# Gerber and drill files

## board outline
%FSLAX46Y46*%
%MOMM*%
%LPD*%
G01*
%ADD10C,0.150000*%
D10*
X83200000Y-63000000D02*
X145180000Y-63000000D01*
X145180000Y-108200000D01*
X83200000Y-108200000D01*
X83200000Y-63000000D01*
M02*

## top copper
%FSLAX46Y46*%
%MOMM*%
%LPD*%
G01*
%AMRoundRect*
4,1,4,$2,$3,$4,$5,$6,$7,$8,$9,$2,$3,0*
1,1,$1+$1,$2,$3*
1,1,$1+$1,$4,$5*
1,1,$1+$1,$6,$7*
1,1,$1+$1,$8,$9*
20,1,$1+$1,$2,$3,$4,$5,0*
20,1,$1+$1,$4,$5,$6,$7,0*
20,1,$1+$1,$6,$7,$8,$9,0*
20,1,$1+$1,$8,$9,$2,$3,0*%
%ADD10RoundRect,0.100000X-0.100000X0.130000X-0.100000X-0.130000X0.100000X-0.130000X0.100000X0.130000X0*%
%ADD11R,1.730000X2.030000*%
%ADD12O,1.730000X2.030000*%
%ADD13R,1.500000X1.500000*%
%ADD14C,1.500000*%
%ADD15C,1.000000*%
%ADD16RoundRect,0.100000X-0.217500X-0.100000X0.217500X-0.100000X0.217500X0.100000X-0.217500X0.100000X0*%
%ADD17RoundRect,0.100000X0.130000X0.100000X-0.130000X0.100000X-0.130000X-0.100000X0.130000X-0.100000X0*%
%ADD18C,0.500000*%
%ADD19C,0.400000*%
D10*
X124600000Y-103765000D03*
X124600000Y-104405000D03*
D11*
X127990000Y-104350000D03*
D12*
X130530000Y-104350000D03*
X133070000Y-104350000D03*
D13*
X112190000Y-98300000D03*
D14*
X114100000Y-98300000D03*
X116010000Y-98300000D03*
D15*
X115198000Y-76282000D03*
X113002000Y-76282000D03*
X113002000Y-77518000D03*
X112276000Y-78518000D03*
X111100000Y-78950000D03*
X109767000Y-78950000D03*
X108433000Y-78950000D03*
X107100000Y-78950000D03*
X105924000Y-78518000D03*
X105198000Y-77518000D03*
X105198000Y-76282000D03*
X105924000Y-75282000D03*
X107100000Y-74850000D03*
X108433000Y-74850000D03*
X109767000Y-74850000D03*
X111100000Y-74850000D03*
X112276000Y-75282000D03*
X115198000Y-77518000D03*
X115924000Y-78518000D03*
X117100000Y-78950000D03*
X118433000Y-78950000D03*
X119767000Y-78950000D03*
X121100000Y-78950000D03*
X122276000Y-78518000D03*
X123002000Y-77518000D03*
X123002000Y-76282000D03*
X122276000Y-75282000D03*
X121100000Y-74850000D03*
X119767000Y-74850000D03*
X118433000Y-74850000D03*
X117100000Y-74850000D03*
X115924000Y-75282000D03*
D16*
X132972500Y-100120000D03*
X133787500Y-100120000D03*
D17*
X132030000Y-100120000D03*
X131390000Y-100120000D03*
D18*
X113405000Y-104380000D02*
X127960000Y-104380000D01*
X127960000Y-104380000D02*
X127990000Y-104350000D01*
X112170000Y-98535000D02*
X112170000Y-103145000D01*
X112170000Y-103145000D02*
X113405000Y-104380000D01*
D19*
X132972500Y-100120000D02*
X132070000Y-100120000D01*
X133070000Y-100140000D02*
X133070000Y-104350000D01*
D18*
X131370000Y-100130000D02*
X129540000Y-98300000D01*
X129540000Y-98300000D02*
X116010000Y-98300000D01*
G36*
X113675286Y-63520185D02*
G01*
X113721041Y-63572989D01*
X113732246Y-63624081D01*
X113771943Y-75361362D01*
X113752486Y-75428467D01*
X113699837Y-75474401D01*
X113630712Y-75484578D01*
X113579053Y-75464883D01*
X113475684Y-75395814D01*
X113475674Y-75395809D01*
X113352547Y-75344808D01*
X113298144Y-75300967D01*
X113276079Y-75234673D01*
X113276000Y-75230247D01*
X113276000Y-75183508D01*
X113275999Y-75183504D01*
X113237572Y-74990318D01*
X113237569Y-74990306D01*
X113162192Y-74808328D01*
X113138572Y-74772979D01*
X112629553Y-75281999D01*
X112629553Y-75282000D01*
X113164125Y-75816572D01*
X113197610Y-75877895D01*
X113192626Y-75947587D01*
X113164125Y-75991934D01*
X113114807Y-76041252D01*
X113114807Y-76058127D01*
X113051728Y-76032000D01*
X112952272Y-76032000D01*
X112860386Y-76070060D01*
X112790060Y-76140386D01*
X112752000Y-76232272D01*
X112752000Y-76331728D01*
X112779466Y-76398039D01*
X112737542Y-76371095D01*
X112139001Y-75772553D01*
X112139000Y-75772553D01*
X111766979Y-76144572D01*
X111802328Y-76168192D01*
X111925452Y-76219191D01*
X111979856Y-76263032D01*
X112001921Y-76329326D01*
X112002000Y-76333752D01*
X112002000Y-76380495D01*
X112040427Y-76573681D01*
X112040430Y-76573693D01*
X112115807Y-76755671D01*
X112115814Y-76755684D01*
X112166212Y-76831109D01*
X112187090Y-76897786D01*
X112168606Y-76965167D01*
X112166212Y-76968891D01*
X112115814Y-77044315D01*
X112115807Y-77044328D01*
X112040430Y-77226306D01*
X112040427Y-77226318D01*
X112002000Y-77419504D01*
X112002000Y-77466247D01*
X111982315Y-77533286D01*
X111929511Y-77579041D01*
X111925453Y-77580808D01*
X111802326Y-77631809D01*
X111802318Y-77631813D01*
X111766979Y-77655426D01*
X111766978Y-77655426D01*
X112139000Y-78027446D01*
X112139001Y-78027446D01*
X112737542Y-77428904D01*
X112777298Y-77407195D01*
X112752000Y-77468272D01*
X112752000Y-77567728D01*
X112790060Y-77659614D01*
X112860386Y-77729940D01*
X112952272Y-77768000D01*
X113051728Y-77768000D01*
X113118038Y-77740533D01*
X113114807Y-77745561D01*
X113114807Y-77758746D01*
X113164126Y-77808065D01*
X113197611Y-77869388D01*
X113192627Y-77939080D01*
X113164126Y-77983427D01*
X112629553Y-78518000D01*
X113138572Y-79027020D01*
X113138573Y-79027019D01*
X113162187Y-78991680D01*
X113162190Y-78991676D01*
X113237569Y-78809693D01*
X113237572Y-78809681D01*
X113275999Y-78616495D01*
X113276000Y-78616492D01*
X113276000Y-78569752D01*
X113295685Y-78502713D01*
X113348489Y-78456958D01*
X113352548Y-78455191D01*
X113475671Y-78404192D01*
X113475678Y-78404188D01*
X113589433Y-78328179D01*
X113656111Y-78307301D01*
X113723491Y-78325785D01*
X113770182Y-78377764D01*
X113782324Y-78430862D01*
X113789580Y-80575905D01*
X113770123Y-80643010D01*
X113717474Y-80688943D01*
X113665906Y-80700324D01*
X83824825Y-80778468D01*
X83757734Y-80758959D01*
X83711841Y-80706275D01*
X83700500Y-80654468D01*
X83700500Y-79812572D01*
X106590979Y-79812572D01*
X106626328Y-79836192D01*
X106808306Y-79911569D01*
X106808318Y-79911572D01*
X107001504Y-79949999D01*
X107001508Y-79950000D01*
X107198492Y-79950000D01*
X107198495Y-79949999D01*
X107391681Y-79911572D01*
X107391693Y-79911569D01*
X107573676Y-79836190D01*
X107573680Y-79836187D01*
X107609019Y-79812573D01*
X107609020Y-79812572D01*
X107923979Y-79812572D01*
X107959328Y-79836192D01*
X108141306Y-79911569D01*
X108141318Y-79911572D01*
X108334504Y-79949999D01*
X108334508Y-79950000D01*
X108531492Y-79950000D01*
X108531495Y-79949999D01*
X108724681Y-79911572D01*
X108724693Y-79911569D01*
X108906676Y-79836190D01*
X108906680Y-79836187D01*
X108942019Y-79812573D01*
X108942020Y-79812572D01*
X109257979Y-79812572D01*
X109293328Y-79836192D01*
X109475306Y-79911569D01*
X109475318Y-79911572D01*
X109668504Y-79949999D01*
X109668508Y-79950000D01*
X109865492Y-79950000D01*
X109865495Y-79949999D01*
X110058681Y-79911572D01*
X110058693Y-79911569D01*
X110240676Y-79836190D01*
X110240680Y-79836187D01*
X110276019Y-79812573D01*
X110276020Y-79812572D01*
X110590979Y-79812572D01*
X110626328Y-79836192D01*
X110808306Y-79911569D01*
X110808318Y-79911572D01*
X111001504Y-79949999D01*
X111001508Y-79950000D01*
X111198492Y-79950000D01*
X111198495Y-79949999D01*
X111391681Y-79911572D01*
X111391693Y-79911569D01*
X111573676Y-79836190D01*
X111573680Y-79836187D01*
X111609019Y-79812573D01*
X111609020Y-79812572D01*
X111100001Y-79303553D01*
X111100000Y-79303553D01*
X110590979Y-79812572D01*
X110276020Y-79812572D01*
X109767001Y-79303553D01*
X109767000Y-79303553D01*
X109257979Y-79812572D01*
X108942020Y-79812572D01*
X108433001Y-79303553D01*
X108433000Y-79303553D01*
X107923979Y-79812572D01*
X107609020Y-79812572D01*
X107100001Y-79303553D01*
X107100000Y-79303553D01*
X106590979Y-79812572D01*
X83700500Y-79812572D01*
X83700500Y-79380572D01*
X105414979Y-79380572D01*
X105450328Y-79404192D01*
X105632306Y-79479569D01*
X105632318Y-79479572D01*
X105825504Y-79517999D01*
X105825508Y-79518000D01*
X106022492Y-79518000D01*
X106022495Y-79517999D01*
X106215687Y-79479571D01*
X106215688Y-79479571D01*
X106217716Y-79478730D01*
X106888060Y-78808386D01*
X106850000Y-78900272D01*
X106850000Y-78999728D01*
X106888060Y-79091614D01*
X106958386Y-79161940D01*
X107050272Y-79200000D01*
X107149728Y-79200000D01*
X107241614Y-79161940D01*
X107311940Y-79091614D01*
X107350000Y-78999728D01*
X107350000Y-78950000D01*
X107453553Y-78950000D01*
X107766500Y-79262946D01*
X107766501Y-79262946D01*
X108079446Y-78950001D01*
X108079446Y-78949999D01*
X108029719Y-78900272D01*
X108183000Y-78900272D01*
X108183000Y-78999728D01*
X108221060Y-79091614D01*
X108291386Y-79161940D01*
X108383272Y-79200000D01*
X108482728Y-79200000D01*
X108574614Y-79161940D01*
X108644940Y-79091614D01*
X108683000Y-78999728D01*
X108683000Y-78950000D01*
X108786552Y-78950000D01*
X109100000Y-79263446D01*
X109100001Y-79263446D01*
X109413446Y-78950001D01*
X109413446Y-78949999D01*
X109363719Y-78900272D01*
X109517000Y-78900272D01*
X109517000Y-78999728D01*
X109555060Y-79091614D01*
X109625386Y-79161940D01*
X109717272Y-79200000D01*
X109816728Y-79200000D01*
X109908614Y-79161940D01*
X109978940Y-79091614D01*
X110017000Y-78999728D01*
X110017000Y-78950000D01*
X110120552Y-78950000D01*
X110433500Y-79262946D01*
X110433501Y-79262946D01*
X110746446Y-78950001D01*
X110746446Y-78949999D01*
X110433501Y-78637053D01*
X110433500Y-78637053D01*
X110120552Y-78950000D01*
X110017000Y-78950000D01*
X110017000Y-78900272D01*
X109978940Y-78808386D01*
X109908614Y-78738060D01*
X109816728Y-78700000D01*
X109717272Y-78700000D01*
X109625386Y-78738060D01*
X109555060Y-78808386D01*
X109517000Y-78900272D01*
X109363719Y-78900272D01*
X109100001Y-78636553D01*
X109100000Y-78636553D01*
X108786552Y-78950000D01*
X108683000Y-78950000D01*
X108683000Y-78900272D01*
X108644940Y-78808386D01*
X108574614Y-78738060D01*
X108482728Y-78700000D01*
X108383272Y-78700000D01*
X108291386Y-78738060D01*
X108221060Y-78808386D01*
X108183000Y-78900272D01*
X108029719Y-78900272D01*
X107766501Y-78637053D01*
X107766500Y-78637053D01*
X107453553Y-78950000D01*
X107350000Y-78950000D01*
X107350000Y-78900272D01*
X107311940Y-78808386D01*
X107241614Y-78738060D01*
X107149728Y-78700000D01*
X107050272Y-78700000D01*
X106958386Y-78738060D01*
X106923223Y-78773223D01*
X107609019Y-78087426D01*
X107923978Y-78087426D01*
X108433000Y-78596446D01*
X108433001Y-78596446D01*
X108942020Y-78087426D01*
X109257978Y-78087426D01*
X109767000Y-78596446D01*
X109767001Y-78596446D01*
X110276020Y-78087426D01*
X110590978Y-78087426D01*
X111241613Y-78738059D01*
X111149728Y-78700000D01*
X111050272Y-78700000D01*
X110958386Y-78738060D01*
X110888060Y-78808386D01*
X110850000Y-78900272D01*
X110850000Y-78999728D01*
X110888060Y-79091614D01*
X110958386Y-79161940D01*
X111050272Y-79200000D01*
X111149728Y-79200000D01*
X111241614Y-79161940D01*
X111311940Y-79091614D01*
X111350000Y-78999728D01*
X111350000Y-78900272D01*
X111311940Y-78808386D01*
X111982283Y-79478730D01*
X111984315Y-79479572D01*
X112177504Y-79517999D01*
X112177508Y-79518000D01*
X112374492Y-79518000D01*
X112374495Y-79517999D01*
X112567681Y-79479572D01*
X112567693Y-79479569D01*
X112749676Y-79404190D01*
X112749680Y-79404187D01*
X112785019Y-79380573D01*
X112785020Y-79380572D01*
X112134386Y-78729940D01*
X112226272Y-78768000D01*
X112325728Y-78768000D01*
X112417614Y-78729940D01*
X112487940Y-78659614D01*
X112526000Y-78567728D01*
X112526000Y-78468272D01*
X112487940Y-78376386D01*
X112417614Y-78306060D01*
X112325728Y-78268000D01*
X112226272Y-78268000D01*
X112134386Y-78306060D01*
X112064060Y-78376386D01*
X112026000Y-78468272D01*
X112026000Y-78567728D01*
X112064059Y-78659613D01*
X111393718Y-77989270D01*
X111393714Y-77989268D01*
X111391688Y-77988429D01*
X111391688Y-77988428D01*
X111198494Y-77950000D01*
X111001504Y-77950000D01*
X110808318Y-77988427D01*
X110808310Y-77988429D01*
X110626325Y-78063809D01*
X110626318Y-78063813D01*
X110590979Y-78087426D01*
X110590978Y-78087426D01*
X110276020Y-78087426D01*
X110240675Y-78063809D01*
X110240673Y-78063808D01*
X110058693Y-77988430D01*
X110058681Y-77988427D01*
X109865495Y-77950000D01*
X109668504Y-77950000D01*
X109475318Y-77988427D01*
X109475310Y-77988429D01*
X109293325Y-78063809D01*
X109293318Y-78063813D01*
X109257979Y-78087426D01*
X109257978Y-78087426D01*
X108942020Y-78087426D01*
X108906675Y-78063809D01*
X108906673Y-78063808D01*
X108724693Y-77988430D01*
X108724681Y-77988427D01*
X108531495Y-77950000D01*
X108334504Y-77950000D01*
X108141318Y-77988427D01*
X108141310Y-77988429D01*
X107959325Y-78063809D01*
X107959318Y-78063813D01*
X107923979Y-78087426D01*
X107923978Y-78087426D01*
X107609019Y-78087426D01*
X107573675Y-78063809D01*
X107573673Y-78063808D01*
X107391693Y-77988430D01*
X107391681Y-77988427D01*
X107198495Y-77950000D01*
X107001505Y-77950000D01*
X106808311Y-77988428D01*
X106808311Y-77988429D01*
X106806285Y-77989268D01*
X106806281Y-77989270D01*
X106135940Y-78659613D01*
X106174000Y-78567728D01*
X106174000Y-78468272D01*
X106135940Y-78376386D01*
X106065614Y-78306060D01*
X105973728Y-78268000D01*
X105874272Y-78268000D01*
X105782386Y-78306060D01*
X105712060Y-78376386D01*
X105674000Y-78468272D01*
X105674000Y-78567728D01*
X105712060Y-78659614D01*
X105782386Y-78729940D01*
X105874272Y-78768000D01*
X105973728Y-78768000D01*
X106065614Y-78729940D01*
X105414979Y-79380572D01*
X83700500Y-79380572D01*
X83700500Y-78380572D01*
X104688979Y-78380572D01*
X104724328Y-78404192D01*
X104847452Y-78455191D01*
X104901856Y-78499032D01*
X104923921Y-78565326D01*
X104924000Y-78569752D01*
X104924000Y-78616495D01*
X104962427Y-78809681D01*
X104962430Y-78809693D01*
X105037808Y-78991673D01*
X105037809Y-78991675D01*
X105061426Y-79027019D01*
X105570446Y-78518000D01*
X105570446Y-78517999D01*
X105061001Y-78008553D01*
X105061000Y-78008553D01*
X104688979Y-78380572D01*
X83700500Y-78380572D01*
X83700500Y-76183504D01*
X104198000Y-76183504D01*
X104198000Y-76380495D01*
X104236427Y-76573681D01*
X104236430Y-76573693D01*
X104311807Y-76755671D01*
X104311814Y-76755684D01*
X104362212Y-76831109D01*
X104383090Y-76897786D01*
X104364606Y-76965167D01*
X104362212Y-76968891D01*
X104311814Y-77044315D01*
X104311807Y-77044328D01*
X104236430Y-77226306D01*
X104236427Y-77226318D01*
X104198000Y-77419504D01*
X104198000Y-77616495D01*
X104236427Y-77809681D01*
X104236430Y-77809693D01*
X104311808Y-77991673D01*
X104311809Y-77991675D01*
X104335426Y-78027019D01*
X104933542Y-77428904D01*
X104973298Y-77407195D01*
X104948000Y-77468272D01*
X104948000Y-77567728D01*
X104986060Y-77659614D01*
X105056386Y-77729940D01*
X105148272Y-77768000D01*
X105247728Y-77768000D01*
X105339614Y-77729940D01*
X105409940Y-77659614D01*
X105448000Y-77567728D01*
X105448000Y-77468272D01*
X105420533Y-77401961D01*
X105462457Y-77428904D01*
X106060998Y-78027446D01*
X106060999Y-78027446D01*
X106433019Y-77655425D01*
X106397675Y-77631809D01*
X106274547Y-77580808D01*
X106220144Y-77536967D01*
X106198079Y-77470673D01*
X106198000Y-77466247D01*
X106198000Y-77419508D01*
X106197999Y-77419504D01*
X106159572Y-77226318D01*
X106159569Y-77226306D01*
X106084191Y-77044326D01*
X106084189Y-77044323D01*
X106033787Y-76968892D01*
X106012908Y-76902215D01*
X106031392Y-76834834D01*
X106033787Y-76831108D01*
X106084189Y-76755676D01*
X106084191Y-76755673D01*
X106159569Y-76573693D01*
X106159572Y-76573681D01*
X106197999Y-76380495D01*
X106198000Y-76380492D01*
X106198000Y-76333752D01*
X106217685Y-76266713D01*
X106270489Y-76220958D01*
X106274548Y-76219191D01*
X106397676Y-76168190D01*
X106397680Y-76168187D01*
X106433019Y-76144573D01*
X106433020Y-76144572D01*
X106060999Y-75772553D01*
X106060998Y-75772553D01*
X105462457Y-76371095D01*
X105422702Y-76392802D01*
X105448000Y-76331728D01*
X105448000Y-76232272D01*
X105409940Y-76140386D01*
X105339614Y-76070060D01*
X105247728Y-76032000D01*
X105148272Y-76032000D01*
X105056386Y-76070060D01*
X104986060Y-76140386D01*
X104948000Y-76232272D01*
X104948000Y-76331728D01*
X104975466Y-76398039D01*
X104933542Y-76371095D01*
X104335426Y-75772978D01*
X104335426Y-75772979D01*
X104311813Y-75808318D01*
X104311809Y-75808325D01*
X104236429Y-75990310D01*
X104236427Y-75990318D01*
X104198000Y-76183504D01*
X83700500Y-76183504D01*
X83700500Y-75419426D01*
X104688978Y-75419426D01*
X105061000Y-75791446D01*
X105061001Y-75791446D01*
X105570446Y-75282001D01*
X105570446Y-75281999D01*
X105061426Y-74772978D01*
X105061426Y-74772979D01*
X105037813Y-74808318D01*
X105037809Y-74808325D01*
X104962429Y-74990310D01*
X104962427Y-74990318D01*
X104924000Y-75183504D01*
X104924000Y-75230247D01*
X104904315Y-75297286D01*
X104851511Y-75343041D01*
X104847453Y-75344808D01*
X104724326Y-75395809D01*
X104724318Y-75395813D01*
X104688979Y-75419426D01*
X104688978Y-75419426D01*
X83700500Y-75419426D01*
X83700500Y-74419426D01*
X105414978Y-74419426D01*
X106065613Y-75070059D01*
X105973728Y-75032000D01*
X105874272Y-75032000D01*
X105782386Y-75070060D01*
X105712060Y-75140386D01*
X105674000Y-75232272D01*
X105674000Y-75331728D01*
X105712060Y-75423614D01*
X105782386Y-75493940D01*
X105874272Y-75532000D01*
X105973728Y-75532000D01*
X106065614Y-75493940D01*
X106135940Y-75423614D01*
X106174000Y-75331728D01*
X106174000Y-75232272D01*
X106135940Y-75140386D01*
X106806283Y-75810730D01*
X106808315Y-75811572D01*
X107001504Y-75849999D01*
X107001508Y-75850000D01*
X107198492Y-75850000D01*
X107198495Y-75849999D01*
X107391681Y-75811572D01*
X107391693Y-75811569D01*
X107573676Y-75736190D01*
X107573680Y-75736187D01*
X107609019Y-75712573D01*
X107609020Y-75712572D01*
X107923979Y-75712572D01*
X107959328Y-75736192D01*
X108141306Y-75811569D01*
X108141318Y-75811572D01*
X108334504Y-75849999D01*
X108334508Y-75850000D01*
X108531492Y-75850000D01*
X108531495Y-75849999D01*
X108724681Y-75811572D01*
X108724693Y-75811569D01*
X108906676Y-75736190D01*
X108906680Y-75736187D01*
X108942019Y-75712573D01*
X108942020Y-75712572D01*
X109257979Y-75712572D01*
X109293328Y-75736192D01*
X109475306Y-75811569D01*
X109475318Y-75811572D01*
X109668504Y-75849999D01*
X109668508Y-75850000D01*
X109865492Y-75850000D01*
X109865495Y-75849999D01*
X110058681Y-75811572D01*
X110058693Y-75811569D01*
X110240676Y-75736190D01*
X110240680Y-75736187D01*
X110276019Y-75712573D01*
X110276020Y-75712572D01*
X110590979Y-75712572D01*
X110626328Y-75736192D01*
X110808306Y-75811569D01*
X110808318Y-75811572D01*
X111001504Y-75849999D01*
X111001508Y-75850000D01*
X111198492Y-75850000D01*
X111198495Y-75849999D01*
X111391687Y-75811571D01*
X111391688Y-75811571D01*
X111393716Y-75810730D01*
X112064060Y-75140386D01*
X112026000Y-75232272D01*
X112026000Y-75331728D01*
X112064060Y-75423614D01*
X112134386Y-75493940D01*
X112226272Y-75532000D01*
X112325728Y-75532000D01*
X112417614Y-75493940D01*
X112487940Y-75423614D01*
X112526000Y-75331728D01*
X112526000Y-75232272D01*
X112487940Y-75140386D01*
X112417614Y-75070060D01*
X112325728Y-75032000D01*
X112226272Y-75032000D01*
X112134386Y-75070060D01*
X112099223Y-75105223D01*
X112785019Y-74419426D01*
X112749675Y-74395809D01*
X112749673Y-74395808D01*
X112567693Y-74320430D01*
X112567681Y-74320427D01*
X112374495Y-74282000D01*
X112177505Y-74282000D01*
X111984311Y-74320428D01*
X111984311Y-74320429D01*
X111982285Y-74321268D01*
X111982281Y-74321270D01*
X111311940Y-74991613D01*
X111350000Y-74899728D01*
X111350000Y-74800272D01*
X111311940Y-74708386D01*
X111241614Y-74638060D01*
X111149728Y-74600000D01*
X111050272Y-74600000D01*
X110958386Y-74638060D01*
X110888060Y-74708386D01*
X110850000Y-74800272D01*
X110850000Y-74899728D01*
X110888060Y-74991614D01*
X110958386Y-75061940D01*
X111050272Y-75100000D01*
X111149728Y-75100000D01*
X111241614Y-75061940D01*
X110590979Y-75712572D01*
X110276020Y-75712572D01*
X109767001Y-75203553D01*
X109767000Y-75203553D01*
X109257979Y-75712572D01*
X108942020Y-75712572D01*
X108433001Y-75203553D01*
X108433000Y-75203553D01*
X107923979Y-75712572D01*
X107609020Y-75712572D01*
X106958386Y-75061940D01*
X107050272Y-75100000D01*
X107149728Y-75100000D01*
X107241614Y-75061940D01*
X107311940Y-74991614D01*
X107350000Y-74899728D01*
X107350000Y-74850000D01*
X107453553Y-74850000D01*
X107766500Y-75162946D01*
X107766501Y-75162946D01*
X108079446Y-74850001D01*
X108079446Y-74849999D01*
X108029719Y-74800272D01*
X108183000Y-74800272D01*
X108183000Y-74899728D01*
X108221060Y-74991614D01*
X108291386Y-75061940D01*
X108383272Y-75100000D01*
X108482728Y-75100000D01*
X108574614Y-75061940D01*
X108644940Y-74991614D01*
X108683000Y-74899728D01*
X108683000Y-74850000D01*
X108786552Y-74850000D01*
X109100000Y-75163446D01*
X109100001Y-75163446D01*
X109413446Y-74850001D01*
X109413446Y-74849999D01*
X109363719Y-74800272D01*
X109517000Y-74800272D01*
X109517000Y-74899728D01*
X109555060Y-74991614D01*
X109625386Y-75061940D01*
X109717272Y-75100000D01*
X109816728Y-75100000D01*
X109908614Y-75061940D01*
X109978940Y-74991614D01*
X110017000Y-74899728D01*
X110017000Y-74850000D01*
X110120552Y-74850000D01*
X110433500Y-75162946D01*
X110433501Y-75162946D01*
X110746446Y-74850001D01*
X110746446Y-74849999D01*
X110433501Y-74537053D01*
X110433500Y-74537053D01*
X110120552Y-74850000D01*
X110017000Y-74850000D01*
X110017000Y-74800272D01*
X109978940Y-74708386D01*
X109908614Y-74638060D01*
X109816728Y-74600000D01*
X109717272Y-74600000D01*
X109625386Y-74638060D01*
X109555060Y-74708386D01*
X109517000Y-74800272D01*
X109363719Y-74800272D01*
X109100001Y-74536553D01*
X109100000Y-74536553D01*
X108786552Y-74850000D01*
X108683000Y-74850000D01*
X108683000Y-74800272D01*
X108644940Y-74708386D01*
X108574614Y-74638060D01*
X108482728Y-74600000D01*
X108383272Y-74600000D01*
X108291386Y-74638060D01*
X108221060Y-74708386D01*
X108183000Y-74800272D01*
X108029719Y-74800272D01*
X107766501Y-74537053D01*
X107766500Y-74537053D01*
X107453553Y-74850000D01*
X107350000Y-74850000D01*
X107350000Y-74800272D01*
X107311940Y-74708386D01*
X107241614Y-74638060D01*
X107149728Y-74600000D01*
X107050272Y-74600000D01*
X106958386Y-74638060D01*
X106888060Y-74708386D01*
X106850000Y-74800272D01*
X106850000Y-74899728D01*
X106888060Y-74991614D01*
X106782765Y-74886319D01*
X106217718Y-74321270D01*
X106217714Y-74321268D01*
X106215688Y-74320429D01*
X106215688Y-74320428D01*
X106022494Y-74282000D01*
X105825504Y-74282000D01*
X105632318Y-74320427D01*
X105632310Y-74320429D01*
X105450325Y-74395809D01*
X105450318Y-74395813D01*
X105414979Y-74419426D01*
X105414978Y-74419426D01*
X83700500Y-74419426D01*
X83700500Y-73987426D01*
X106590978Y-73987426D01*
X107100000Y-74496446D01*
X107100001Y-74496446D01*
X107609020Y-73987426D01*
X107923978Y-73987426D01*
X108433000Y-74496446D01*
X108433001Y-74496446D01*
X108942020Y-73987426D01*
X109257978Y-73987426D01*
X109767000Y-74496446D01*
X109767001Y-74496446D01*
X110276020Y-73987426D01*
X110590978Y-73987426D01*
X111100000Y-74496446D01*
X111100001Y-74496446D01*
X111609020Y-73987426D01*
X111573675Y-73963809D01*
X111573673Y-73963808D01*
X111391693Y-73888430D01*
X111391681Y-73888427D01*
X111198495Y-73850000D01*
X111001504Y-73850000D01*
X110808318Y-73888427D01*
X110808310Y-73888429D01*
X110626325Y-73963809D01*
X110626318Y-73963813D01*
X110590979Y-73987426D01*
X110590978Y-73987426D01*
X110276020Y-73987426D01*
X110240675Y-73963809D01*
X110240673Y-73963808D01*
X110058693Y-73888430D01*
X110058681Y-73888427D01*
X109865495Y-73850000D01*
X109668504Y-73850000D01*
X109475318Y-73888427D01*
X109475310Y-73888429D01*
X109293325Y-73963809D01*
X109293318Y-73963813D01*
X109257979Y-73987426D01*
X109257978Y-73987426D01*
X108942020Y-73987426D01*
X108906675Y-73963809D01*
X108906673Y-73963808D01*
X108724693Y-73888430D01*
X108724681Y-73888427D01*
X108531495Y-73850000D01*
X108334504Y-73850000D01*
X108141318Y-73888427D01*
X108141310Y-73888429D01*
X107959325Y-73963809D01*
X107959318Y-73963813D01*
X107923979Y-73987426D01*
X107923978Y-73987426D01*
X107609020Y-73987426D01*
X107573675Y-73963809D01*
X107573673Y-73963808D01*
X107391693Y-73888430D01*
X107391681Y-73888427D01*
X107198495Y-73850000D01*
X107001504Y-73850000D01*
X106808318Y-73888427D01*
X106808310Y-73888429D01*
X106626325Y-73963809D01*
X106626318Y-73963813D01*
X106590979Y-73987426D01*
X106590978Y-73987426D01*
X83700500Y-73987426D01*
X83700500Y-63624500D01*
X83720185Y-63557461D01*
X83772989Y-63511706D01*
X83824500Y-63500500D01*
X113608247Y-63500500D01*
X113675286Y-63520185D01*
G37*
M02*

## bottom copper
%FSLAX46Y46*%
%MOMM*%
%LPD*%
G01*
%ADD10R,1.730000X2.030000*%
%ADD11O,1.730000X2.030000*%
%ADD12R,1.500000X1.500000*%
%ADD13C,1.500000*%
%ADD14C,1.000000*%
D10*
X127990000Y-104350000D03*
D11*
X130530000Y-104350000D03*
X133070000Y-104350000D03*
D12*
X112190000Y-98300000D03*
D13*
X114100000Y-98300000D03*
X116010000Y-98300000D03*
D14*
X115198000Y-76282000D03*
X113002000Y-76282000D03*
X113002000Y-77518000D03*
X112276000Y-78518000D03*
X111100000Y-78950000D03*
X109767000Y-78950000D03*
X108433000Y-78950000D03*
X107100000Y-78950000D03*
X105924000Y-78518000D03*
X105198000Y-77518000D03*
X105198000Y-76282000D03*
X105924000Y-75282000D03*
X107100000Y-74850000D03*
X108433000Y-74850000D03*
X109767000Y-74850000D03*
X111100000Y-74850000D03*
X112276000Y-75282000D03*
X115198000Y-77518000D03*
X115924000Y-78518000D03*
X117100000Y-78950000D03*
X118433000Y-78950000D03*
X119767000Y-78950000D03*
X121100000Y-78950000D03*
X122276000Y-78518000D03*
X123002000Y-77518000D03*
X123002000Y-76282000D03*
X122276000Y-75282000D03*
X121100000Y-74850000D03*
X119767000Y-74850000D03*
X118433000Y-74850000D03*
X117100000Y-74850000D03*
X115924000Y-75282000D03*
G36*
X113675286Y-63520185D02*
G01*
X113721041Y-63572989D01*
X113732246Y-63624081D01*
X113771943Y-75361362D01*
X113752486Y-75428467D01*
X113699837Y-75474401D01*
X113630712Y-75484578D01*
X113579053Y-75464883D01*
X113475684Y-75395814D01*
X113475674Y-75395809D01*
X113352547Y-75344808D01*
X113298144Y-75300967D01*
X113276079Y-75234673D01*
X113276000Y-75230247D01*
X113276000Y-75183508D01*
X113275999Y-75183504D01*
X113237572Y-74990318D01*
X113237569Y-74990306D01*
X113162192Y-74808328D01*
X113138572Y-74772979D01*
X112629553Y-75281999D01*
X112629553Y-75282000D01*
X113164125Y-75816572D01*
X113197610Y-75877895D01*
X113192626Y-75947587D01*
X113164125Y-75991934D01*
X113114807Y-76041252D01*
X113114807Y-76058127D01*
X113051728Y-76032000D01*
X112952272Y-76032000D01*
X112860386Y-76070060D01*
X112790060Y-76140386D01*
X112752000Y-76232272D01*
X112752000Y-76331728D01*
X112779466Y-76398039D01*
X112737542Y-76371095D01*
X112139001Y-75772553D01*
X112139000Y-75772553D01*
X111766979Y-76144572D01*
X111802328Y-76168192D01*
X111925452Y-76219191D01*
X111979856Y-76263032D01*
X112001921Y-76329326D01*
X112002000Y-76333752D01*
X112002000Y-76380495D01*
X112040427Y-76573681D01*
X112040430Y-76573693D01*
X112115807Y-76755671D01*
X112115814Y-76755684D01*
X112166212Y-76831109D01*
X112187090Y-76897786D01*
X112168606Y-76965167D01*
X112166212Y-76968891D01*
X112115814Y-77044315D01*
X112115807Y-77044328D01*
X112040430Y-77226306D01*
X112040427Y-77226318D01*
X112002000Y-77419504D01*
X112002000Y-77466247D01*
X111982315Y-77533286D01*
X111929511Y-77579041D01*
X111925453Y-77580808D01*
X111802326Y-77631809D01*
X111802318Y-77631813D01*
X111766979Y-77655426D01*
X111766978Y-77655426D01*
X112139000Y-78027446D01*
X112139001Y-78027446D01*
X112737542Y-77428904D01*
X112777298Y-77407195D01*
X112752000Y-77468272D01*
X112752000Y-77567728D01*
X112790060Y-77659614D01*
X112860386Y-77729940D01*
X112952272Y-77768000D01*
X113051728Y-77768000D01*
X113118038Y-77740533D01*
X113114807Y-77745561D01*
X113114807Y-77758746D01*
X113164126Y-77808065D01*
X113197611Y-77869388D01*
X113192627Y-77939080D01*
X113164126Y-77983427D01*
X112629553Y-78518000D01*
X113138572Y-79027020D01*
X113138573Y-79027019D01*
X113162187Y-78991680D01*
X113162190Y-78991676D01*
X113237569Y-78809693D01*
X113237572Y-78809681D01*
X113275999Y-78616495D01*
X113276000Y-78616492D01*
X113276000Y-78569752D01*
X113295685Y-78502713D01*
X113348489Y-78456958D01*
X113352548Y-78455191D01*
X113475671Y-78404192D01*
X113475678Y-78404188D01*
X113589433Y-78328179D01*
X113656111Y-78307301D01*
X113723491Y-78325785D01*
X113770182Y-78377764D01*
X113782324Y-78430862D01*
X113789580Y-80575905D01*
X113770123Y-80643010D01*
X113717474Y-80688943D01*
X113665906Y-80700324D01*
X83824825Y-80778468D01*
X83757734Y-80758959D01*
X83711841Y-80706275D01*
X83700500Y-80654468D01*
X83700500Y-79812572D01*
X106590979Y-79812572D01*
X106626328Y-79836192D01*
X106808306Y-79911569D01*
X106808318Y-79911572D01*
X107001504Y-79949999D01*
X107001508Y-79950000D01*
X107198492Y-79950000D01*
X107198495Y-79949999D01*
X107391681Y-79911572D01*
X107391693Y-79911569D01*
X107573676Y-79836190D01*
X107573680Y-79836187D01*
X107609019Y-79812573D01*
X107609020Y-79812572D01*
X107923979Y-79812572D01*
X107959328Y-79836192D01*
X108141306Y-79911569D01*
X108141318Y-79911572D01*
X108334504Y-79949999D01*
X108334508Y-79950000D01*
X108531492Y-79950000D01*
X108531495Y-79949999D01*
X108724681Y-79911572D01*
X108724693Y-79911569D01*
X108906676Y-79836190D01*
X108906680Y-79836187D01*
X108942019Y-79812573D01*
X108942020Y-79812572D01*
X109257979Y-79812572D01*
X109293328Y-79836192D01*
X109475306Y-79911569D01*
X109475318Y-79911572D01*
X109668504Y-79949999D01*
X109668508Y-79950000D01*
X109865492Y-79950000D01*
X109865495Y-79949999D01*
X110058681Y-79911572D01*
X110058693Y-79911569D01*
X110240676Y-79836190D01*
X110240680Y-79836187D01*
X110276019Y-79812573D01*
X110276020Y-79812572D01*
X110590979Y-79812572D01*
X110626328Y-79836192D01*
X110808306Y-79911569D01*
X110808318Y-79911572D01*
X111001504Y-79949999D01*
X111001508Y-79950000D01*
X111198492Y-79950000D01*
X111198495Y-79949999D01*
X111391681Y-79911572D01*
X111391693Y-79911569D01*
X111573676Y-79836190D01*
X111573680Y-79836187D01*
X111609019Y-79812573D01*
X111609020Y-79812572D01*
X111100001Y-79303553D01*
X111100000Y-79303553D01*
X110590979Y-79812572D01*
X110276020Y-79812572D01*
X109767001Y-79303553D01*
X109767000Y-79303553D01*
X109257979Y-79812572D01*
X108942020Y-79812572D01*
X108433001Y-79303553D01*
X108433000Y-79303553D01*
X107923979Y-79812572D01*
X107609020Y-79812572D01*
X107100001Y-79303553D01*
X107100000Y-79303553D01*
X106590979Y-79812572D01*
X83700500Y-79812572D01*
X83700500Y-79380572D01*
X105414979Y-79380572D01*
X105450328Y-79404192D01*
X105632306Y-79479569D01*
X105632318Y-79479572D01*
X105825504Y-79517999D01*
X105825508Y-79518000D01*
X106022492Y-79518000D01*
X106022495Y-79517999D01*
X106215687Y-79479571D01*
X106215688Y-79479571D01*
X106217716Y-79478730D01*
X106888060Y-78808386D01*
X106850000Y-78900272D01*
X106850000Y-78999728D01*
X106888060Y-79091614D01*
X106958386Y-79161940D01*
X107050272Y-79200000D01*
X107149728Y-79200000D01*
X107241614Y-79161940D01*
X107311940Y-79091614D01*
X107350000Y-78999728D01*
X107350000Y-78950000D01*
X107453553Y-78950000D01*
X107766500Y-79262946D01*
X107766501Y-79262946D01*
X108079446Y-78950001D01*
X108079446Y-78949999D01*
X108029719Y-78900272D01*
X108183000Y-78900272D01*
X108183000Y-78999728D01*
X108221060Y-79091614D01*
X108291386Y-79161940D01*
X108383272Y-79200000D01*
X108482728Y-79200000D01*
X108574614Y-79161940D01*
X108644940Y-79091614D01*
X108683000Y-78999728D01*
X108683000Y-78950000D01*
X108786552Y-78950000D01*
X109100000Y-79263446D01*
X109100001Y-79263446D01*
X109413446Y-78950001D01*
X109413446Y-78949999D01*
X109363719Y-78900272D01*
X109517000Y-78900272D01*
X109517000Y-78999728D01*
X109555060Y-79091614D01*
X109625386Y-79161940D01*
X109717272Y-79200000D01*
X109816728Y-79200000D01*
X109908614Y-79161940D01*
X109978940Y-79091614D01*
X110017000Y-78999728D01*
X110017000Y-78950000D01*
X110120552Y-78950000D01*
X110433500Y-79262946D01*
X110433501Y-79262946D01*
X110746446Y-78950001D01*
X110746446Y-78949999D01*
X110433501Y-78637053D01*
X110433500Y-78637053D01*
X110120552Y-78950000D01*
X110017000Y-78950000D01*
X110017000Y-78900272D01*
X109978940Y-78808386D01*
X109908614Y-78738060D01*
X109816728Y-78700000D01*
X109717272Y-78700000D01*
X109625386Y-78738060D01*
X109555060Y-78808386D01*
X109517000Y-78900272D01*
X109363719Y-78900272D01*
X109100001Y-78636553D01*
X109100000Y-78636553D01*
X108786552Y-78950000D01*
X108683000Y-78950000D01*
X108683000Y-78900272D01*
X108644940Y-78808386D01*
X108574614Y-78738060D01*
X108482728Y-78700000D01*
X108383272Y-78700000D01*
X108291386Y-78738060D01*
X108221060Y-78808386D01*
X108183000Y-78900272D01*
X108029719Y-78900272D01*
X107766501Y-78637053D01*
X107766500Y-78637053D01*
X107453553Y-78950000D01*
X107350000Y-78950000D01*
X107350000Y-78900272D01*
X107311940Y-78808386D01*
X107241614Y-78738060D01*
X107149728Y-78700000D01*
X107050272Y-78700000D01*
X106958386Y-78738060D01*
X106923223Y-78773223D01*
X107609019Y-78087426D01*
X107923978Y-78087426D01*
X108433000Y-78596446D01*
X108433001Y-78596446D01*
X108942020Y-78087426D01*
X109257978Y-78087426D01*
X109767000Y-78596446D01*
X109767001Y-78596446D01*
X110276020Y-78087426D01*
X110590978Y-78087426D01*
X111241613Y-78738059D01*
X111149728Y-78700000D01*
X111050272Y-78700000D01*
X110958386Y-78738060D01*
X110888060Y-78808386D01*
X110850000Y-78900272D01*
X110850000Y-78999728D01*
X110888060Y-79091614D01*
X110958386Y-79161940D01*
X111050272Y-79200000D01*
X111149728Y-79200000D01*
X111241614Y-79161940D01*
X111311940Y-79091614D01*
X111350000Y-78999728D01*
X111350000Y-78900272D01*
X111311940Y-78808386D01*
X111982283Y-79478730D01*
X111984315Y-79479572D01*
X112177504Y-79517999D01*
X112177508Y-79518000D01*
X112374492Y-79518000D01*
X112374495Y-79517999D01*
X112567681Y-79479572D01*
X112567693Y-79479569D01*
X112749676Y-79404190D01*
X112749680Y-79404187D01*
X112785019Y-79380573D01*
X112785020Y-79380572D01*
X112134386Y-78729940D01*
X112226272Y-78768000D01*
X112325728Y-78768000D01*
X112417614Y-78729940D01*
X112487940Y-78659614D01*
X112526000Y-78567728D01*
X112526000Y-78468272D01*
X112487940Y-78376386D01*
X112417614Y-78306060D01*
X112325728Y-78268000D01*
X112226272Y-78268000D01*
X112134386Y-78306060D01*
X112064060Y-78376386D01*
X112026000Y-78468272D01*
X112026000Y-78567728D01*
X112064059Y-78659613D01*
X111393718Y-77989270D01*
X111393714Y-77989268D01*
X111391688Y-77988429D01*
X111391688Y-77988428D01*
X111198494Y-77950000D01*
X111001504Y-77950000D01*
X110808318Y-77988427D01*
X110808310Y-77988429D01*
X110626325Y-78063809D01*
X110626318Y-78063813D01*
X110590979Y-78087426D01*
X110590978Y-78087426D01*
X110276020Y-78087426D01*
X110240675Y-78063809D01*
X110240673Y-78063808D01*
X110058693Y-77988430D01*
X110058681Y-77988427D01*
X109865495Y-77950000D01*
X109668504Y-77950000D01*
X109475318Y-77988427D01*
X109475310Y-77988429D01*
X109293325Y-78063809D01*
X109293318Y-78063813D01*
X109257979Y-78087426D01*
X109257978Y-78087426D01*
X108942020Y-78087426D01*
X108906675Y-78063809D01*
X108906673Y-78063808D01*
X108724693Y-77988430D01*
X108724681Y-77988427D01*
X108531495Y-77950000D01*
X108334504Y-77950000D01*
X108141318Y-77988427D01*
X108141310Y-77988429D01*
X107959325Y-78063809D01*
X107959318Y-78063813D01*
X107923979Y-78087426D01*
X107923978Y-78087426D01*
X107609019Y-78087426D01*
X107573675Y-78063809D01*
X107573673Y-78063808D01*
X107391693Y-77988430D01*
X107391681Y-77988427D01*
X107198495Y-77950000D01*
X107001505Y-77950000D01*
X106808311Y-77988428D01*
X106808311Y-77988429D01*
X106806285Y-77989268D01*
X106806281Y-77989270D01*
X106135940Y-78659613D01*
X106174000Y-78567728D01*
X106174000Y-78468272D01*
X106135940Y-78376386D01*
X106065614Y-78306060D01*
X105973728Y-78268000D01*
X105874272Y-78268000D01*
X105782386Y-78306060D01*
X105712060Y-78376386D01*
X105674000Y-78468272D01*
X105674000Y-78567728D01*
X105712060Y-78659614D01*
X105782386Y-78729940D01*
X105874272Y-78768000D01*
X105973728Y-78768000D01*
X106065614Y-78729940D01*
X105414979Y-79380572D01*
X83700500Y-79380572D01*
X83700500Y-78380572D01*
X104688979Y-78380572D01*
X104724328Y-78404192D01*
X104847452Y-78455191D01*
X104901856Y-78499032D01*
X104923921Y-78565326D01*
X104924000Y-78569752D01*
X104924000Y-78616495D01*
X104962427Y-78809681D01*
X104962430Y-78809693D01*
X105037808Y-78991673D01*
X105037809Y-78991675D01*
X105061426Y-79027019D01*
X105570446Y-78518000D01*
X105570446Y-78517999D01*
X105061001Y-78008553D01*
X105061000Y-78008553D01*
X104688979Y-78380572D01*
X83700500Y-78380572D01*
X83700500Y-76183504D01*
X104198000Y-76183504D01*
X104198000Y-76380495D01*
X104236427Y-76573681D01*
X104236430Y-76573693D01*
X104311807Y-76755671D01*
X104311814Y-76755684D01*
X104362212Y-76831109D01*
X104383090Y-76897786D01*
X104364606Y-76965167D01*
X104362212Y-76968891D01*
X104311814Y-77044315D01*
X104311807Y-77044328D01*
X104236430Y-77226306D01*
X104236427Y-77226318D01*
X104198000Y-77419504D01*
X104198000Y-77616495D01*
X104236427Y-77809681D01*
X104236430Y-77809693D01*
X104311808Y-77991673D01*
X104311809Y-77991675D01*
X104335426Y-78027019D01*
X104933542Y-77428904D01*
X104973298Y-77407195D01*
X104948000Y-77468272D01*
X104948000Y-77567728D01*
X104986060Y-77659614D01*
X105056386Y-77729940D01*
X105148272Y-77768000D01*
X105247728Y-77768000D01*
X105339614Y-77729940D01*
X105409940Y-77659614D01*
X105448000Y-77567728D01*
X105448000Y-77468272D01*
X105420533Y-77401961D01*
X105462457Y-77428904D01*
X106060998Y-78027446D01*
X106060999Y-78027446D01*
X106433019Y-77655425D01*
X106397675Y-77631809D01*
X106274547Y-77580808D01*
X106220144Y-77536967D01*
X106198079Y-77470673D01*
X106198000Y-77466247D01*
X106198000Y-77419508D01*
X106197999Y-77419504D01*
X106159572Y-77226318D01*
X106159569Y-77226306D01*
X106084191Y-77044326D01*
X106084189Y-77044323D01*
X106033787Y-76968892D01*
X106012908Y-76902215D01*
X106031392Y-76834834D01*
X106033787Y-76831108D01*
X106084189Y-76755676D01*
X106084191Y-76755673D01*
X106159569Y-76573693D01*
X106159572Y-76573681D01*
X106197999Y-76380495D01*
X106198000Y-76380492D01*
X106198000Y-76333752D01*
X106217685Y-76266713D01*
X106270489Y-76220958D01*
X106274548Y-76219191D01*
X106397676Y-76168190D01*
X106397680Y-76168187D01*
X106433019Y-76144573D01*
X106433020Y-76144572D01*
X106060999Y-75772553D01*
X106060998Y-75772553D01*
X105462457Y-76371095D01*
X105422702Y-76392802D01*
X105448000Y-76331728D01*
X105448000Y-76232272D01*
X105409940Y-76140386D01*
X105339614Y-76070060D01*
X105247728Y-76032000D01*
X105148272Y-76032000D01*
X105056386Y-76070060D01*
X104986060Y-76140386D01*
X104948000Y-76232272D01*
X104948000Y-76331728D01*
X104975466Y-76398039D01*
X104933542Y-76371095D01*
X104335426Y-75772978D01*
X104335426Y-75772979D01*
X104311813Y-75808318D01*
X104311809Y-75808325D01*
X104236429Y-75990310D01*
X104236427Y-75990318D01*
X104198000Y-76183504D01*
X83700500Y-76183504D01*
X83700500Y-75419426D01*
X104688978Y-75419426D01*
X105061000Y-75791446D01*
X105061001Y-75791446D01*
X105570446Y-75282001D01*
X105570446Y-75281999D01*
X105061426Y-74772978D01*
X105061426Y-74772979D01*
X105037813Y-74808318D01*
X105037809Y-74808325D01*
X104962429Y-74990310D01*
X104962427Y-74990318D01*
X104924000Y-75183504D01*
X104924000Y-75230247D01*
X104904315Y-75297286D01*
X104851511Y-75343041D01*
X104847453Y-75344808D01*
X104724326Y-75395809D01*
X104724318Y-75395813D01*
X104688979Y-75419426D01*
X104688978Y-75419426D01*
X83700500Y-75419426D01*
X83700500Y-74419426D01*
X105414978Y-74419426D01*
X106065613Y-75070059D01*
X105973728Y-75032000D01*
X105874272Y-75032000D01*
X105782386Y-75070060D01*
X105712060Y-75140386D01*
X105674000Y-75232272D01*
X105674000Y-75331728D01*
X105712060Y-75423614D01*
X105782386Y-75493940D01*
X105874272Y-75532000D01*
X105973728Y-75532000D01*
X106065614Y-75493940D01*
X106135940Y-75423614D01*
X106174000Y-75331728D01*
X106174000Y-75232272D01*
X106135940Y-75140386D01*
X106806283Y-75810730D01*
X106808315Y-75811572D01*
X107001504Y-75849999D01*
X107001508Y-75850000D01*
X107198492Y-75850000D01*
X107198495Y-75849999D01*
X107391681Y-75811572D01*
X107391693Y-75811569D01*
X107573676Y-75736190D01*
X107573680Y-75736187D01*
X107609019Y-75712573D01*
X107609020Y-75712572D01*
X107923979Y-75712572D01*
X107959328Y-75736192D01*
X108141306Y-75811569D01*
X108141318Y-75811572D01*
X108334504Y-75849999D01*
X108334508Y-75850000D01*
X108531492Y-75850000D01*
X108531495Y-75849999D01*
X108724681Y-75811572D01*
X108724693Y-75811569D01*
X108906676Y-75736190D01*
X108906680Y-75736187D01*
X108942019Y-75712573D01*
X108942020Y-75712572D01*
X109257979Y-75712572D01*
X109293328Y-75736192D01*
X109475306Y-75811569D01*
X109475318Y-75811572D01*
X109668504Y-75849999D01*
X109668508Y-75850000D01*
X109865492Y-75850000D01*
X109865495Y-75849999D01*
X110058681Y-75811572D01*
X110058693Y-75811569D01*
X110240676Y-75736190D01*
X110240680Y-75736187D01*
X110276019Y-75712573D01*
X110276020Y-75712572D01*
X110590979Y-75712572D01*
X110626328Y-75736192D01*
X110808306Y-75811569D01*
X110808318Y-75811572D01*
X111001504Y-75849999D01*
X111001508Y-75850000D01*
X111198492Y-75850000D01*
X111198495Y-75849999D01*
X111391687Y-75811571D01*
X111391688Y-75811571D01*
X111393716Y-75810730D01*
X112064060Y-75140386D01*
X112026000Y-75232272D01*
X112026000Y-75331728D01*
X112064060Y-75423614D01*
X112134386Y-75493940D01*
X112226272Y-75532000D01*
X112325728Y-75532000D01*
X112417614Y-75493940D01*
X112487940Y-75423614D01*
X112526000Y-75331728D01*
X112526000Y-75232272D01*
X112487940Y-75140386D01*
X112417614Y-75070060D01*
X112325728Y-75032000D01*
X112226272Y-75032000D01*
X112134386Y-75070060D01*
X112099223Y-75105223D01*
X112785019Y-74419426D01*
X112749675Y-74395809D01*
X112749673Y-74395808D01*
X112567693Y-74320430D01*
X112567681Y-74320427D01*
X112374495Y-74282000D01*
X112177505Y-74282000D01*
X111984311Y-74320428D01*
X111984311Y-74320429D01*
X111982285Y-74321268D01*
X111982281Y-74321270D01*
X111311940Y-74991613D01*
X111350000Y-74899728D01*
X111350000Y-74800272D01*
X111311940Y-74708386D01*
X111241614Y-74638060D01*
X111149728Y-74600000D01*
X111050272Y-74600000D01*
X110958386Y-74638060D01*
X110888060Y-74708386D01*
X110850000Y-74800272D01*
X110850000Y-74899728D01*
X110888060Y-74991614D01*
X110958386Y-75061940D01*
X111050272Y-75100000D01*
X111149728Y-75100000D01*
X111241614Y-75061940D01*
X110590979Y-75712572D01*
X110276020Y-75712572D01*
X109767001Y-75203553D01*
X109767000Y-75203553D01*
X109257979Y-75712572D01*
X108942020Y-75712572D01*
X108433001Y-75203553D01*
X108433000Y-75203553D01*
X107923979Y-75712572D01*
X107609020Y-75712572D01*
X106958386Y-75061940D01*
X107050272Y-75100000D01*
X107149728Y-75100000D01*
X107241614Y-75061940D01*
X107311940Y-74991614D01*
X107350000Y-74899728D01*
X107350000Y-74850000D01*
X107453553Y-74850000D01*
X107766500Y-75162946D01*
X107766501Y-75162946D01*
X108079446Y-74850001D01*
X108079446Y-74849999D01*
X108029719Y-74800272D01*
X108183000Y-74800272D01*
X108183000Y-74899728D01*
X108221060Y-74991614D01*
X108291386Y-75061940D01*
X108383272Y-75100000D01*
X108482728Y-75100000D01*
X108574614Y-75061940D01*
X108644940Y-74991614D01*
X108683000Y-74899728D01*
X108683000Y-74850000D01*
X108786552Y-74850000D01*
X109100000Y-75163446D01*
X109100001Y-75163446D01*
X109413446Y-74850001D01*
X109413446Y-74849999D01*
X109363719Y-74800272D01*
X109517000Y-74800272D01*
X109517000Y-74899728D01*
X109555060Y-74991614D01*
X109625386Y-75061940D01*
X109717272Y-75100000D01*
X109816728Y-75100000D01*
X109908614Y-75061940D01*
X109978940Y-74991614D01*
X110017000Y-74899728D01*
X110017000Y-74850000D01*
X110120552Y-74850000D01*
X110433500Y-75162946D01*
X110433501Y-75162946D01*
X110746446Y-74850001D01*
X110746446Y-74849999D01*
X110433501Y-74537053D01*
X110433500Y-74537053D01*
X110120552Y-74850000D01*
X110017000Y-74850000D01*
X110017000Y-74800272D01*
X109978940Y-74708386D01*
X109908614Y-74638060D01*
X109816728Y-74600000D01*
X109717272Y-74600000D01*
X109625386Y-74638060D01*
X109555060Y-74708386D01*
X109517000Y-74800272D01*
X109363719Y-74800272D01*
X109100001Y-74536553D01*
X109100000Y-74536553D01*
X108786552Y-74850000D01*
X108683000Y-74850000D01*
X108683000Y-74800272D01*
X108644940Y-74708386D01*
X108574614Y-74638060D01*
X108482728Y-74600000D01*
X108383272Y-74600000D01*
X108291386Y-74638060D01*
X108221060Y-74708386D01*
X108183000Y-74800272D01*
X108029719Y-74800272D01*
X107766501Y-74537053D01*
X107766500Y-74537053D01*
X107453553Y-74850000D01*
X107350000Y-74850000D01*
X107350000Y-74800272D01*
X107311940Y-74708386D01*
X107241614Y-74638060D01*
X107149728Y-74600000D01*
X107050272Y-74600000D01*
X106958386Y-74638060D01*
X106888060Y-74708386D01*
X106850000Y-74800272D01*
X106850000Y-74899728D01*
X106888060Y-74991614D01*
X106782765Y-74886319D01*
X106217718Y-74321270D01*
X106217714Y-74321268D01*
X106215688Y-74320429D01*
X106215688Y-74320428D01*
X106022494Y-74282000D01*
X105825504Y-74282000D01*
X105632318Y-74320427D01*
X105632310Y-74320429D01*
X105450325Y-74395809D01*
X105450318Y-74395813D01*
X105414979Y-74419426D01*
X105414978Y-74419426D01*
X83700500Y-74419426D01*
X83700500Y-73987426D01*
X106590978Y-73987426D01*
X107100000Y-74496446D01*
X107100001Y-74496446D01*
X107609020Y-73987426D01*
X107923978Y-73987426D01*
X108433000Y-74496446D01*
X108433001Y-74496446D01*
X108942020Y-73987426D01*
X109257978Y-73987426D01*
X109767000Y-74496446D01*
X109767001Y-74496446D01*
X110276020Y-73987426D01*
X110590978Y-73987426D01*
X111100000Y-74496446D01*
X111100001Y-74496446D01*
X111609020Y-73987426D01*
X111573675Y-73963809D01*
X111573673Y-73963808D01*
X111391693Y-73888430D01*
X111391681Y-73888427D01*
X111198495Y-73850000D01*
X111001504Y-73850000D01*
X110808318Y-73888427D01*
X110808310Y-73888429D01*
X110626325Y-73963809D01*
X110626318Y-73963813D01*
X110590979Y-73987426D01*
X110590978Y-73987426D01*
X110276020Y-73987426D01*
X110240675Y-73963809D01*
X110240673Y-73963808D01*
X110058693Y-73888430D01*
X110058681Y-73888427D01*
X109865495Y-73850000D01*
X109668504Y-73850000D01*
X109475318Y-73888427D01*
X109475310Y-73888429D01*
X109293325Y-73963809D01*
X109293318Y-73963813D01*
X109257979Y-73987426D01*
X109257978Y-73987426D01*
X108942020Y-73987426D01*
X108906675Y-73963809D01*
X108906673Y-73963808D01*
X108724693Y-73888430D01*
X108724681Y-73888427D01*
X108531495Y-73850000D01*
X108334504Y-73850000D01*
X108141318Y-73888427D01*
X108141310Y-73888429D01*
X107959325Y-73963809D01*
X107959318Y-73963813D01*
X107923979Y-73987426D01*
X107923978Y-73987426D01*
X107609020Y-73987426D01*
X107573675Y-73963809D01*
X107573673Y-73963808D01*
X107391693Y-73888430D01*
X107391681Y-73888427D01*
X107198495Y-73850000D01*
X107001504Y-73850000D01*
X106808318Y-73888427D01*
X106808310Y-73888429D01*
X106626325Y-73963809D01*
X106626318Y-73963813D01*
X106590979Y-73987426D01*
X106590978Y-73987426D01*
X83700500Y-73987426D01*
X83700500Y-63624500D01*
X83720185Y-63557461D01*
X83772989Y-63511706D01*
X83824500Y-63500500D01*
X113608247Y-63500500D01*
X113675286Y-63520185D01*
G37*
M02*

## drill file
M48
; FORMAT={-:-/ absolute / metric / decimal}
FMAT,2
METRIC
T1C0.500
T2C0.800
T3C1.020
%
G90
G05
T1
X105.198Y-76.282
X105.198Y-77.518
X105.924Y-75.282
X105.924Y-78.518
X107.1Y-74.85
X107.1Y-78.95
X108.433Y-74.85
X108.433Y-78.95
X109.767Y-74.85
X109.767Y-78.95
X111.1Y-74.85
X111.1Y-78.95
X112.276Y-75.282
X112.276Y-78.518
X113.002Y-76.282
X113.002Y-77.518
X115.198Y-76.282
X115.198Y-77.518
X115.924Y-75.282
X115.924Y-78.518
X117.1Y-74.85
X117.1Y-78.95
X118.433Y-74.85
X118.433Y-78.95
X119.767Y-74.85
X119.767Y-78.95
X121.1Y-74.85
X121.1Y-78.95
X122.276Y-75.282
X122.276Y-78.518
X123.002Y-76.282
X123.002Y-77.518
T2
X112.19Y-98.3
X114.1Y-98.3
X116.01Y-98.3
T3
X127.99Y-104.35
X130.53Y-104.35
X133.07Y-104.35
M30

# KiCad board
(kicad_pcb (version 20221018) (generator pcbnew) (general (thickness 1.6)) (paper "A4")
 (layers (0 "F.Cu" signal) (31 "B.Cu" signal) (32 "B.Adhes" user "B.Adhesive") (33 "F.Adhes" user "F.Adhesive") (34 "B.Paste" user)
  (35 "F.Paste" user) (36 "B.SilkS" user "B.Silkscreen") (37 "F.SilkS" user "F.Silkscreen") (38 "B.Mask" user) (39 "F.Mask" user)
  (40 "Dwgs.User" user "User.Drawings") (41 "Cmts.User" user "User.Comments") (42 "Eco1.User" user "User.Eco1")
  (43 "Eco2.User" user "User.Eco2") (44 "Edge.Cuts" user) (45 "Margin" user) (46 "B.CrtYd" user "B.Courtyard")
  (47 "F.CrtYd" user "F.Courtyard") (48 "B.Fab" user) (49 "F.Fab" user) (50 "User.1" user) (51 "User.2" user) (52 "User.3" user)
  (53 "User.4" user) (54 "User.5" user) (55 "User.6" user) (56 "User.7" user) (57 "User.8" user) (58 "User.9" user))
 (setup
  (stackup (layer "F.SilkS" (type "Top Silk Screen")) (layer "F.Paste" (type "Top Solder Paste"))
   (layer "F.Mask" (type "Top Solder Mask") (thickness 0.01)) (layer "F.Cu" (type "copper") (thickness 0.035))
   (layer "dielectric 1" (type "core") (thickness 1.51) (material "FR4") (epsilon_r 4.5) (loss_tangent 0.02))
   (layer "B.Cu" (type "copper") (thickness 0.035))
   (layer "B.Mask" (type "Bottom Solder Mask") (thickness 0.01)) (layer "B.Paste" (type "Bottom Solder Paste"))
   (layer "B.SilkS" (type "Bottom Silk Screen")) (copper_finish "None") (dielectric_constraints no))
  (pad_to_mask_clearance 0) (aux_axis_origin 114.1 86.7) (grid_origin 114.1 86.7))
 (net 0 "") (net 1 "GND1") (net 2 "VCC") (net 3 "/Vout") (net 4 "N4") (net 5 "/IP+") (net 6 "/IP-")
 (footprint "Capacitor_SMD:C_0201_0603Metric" (layer "F.Cu") (at 124.6 104.085 -90)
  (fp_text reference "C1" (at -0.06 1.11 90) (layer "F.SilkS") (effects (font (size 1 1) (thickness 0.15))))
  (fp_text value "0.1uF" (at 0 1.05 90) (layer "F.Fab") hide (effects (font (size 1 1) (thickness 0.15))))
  (pad "" smd roundrect (at -0.345 0 270) (size 0.318 0.36) (layers "F.Paste") (roundrect_rratio 0.25))
  (pad "" smd roundrect (at 0.345 0 270) (size 0.318 0.36) (layers "F.Paste") (roundrect_rratio 0.25))
  (pad "1" smd roundrect (at -0.32 0 270) (size 0.46 0.4) (layers "F.Cu" "F.Mask") (roundrect_rratio 0.25) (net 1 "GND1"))
  (pad "2" smd roundrect (at 0.32 0 270) (size 0.46 0.4) (layers "F.Cu" "F.Mask") (roundrect_rratio 0.25) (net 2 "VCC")))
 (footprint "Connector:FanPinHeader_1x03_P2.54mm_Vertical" (layer "F.Cu") (at 127.99 104.35)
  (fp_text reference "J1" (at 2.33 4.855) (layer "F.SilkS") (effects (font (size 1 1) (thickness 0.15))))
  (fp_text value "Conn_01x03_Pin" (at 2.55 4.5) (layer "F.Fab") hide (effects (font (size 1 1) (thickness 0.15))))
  (pad "1" thru_hole rect (at 0 0 90) (size 2.03 1.73) (drill 1.02) (layers "*.Cu" "*.Mask") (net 2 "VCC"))
  (pad "2" thru_hole oval (at 2.54 0 90) (size 2.03 1.73) (drill 1.02) (layers "*.Cu" "*.Mask") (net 1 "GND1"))
  (pad "3" thru_hole oval (at 5.08 0 90) (size 2.03 1.73) (drill 1.02) (layers "*.Cu" "*.Mask") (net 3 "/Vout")))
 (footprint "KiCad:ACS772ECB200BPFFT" (layer "F.Cu") (at 112.19 98.3)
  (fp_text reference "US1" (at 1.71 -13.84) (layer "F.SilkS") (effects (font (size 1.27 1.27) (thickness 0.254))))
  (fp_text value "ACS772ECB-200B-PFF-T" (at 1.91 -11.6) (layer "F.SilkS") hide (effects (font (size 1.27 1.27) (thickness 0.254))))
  (pad "1" thru_hole rect (at 0 0) (size 1.5 1.5) (drill 0.8) (layers "*.Cu" "*.Mask") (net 2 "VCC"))
  (pad "2" thru_hole circle (at 1.91 0) (size 1.5 1.5) (drill 0.8) (layers "*.Cu" "*.Mask") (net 1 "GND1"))
  (pad "3" thru_hole circle (at 3.82 0) (size 1.5 1.5) (drill 0.8) (layers "*.Cu" "*.Mask") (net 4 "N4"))
  (pad "4" thru_hole circle (at 3.008 -22.018) (size 1 1) (drill 0.5) (layers "*.Cu" "*.Mask") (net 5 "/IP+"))
  (pad "5" thru_hole circle (at 0.812 -22.018) (size 1 1) (drill 0.5) (layers "*.Cu" "*.Mask") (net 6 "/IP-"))
  (pad "6" thru_hole circle (at 0.812 -20.782) (size 1 1) (drill 0.5) (layers "*.Cu" "*.Mask") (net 6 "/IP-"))
  (pad "7" thru_hole circle (at 0.086 -19.782) (size 1 1) (drill 0.5) (layers "*.Cu" "*.Mask") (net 6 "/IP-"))
  (pad "8" thru_hole circle (at -1.09 -19.35) (size 1 1) (drill 0.5) (layers "*.Cu" "*.Mask") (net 6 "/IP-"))
  (pad "9" thru_hole circle (at -2.423 -19.35) (size 1 1) (drill 0.5) (layers "*.Cu" "*.Mask") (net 6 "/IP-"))
  (pad "10" thru_hole circle (at -3.757 -19.35) (size 1 1) (drill 0.5) (layers "*.Cu" "*.Mask") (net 6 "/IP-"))
  (pad "11" thru_hole circle (at -5.09 -19.35) (size 1 1) (drill 0.5) (layers "*.Cu" "*.Mask") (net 6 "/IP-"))
  (pad "12" thru_hole circle (at -6.266 -19.782) (size 1 1) (drill 0.5) (layers "*.Cu" "*.Mask") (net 6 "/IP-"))
  (pad "13" thru_hole circle (at -6.992 -20.782) (size 1 1) (drill 0.5) (layers "*.Cu" "*.Mask") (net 6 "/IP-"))
  (pad "14" thru_hole circle (at -6.992 -22.018) (size 1 1) (drill 0.5) (layers "*.Cu" "*.Mask") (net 6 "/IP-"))
  (pad "15" thru_hole circle (at -6.266 -23.018) (size 1 1) (drill 0.5) (layers "*.Cu" "*.Mask") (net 6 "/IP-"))
  (pad "16" thru_hole circle (at -5.09 -23.45) (size 1 1) (drill 0.5) (layers "*.Cu" "*.Mask") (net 6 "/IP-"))
  (pad "17" thru_hole circle (at -3.757 -23.45) (size 1 1) (drill 0.5) (layers "*.Cu" "*.Mask") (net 6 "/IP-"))
  (pad "18" thru_hole circle (at -2.423 -23.45) (size 1 1) (drill 0.5) (layers "*.Cu" "*.Mask") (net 6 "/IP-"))
  (pad "19" thru_hole circle (at -1.09 -23.45) (size 1 1) (drill 0.5) (layers "*.Cu" "*.Mask") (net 6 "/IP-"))
  (pad "20" thru_hole circle (at 0.086 -23.018) (size 1 1) (drill 0.5) (layers "*.Cu" "*.Mask") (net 6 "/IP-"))
  (pad "21" thru_hole circle (at 3.008 -20.782) (size 1 1) (drill 0.5) (layers "*.Cu" "*.Mask") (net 5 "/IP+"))
  (pad "22" thru_hole circle (at 3.734 -19.782) (size 1 1) (drill 0.5) (layers "*.Cu" "*.Mask") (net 5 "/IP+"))
  (pad "23" thru_hole circle (at 4.91 -19.35) (size 1 1) (drill 0.5) (layers "*.Cu" "*.Mask") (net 5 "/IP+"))
  (pad "24" thru_hole circle (at 6.243 -19.35) (size 1 1) (drill 0.5) (layers "*.Cu" "*.Mask") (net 5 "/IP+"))
  (pad "25" thru_hole circle (at 7.577 -19.35) (size 1 1) (drill 0.5) (layers "*.Cu" "*.Mask") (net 5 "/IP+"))
  (pad "26" thru_hole circle (at 8.91 -19.35) (size 1 1) (drill 0.5) (layers "*.Cu" "*.Mask") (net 5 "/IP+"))
  (pad "27" thru_hole circle (at 10.086 -19.782) (size 1 1) (drill 0.5) (layers "*.Cu" "*.Mask") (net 5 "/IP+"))
  (pad "28" thru_hole circle (at 10.812 -20.782) (size 1 1) (drill 0.5) (layers "*.Cu" "*.Mask") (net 5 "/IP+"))
  (pad "29" thru_hole circle (at 10.812 -22.018) (size 1 1) (drill 0.5) (layers "*.Cu" "*.Mask") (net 5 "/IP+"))
  (pad "30" thru_hole circle (at 10.086 -23.018) (size 1 1) (drill 0.5) (layers "*.Cu" "*.Mask") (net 5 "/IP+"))
  (pad "31" thru_hole circle (at 8.91 -23.45) (size 1 1) (drill 0.5) (layers "*.Cu" "*.Mask") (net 5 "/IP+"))
  (pad "32" thru_hole circle (at 7.577 -23.45) (size 1 1) (drill 0.5) (layers "*.Cu" "*.Mask") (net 5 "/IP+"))
  (pad "33" thru_hole circle (at 6.243 -23.45) (size 1 1) (drill 0.5) (layers "*.Cu" "*.Mask") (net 5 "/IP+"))
  (pad "34" thru_hole circle (at 4.91 -23.45) (size 1 1) (drill 0.5) (layers "*.Cu" "*.Mask") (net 5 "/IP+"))
  (pad "35" thru_hole circle (at 3.734 -23.018) (size 1 1) (drill 0.5) (layers "*.Cu" "*.Mask") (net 5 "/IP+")))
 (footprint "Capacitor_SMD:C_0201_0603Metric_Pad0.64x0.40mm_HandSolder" (layer "F.Cu") (at 133.38 100.12)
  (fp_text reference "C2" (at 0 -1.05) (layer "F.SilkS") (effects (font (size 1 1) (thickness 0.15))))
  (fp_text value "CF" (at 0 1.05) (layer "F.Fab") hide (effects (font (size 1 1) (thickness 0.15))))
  (pad "" smd roundrect (at -0.4325 0) (size 0.458 0.36) (layers "F.Paste") (roundrect_rratio 0.25))
  (pad "" smd roundrect (at 0.4325 0) (size 0.458 0.36) (layers "F.Paste") (roundrect_rratio 0.25))
  (pad "1" smd roundrect (at -0.4075 0) (size 0.635 0.4) (layers "F.Cu" "F.Mask") (roundrect_rratio 0.25) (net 3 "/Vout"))
  (pad "2" smd roundrect (at 0.4075 0) (size 0.635 0.4) (layers "F.Cu" "F.Mask") (roundrect_rratio 0.25) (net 1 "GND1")))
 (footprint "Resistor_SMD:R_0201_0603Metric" (layer "F.Cu") (at 131.71 100.12 180)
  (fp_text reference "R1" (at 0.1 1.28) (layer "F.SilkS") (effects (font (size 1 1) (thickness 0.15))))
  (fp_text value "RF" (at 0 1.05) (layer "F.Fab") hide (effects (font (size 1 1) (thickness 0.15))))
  (pad "" smd roundrect (at -0.345 0 180) (size 0.318 0.36) (layers "F.Paste") (roundrect_rratio 0.25))
  (pad "" smd roundrect (at 0.345 0 180) (size 0.318 0.36) (layers "F.Paste") (roundrect_rratio 0.25))
  (pad "1" smd roundrect (at -0.32 0 180) (size 0.46 0.4) (layers "F.Cu" "F.Mask") (roundrect_rratio 0.25) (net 3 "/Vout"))
  (pad "2" smd roundrect (at 0.32 0 180) (size 0.46 0.4) (layers "F.Cu" "F.Mask") (roundrect_rratio 0.25) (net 4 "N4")))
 (gr_rect (start 83.2 63) (end 145.18 108.2) (stroke (width 0.15) (type default)) (fill none) (layer "Edge.Cuts"))
 (segment (start 113.405 104.38) (end 127.96 104.38) (width 0.5) (layer "F.Cu") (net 2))
 (segment (start 127.96 104.38) (end 127.99 104.35) (width 0.5) (layer "F.Cu") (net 2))
 (segment (start 112.17 98.535) (end 112.17 103.145) (width 0.5) (layer "F.Cu") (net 2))
 (segment (start 112.17 103.145) (end 113.405 104.38) (width 0.5) (layer "F.Cu") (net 2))
 (segment (start 132.9725 100.12) (end 132.07 100.12) (width 0.4) (layer "F.Cu") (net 3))
 (segment (start 133.07 100.14) (end 133.07 104.35) (width 0.4) (layer "F.Cu") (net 3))
 (segment (start 131.37 100.13) (end 129.54 98.3) (width 0.5) (layer "F.Cu") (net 4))
 (segment (start 129.54 98.3) (end 116.01 98.3) (width 0.5) (layer "F.Cu") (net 4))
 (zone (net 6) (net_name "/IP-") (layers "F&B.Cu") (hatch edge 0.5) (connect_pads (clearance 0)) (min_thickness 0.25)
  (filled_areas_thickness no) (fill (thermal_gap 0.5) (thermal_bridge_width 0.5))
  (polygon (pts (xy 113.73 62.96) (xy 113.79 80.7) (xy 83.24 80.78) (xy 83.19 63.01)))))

